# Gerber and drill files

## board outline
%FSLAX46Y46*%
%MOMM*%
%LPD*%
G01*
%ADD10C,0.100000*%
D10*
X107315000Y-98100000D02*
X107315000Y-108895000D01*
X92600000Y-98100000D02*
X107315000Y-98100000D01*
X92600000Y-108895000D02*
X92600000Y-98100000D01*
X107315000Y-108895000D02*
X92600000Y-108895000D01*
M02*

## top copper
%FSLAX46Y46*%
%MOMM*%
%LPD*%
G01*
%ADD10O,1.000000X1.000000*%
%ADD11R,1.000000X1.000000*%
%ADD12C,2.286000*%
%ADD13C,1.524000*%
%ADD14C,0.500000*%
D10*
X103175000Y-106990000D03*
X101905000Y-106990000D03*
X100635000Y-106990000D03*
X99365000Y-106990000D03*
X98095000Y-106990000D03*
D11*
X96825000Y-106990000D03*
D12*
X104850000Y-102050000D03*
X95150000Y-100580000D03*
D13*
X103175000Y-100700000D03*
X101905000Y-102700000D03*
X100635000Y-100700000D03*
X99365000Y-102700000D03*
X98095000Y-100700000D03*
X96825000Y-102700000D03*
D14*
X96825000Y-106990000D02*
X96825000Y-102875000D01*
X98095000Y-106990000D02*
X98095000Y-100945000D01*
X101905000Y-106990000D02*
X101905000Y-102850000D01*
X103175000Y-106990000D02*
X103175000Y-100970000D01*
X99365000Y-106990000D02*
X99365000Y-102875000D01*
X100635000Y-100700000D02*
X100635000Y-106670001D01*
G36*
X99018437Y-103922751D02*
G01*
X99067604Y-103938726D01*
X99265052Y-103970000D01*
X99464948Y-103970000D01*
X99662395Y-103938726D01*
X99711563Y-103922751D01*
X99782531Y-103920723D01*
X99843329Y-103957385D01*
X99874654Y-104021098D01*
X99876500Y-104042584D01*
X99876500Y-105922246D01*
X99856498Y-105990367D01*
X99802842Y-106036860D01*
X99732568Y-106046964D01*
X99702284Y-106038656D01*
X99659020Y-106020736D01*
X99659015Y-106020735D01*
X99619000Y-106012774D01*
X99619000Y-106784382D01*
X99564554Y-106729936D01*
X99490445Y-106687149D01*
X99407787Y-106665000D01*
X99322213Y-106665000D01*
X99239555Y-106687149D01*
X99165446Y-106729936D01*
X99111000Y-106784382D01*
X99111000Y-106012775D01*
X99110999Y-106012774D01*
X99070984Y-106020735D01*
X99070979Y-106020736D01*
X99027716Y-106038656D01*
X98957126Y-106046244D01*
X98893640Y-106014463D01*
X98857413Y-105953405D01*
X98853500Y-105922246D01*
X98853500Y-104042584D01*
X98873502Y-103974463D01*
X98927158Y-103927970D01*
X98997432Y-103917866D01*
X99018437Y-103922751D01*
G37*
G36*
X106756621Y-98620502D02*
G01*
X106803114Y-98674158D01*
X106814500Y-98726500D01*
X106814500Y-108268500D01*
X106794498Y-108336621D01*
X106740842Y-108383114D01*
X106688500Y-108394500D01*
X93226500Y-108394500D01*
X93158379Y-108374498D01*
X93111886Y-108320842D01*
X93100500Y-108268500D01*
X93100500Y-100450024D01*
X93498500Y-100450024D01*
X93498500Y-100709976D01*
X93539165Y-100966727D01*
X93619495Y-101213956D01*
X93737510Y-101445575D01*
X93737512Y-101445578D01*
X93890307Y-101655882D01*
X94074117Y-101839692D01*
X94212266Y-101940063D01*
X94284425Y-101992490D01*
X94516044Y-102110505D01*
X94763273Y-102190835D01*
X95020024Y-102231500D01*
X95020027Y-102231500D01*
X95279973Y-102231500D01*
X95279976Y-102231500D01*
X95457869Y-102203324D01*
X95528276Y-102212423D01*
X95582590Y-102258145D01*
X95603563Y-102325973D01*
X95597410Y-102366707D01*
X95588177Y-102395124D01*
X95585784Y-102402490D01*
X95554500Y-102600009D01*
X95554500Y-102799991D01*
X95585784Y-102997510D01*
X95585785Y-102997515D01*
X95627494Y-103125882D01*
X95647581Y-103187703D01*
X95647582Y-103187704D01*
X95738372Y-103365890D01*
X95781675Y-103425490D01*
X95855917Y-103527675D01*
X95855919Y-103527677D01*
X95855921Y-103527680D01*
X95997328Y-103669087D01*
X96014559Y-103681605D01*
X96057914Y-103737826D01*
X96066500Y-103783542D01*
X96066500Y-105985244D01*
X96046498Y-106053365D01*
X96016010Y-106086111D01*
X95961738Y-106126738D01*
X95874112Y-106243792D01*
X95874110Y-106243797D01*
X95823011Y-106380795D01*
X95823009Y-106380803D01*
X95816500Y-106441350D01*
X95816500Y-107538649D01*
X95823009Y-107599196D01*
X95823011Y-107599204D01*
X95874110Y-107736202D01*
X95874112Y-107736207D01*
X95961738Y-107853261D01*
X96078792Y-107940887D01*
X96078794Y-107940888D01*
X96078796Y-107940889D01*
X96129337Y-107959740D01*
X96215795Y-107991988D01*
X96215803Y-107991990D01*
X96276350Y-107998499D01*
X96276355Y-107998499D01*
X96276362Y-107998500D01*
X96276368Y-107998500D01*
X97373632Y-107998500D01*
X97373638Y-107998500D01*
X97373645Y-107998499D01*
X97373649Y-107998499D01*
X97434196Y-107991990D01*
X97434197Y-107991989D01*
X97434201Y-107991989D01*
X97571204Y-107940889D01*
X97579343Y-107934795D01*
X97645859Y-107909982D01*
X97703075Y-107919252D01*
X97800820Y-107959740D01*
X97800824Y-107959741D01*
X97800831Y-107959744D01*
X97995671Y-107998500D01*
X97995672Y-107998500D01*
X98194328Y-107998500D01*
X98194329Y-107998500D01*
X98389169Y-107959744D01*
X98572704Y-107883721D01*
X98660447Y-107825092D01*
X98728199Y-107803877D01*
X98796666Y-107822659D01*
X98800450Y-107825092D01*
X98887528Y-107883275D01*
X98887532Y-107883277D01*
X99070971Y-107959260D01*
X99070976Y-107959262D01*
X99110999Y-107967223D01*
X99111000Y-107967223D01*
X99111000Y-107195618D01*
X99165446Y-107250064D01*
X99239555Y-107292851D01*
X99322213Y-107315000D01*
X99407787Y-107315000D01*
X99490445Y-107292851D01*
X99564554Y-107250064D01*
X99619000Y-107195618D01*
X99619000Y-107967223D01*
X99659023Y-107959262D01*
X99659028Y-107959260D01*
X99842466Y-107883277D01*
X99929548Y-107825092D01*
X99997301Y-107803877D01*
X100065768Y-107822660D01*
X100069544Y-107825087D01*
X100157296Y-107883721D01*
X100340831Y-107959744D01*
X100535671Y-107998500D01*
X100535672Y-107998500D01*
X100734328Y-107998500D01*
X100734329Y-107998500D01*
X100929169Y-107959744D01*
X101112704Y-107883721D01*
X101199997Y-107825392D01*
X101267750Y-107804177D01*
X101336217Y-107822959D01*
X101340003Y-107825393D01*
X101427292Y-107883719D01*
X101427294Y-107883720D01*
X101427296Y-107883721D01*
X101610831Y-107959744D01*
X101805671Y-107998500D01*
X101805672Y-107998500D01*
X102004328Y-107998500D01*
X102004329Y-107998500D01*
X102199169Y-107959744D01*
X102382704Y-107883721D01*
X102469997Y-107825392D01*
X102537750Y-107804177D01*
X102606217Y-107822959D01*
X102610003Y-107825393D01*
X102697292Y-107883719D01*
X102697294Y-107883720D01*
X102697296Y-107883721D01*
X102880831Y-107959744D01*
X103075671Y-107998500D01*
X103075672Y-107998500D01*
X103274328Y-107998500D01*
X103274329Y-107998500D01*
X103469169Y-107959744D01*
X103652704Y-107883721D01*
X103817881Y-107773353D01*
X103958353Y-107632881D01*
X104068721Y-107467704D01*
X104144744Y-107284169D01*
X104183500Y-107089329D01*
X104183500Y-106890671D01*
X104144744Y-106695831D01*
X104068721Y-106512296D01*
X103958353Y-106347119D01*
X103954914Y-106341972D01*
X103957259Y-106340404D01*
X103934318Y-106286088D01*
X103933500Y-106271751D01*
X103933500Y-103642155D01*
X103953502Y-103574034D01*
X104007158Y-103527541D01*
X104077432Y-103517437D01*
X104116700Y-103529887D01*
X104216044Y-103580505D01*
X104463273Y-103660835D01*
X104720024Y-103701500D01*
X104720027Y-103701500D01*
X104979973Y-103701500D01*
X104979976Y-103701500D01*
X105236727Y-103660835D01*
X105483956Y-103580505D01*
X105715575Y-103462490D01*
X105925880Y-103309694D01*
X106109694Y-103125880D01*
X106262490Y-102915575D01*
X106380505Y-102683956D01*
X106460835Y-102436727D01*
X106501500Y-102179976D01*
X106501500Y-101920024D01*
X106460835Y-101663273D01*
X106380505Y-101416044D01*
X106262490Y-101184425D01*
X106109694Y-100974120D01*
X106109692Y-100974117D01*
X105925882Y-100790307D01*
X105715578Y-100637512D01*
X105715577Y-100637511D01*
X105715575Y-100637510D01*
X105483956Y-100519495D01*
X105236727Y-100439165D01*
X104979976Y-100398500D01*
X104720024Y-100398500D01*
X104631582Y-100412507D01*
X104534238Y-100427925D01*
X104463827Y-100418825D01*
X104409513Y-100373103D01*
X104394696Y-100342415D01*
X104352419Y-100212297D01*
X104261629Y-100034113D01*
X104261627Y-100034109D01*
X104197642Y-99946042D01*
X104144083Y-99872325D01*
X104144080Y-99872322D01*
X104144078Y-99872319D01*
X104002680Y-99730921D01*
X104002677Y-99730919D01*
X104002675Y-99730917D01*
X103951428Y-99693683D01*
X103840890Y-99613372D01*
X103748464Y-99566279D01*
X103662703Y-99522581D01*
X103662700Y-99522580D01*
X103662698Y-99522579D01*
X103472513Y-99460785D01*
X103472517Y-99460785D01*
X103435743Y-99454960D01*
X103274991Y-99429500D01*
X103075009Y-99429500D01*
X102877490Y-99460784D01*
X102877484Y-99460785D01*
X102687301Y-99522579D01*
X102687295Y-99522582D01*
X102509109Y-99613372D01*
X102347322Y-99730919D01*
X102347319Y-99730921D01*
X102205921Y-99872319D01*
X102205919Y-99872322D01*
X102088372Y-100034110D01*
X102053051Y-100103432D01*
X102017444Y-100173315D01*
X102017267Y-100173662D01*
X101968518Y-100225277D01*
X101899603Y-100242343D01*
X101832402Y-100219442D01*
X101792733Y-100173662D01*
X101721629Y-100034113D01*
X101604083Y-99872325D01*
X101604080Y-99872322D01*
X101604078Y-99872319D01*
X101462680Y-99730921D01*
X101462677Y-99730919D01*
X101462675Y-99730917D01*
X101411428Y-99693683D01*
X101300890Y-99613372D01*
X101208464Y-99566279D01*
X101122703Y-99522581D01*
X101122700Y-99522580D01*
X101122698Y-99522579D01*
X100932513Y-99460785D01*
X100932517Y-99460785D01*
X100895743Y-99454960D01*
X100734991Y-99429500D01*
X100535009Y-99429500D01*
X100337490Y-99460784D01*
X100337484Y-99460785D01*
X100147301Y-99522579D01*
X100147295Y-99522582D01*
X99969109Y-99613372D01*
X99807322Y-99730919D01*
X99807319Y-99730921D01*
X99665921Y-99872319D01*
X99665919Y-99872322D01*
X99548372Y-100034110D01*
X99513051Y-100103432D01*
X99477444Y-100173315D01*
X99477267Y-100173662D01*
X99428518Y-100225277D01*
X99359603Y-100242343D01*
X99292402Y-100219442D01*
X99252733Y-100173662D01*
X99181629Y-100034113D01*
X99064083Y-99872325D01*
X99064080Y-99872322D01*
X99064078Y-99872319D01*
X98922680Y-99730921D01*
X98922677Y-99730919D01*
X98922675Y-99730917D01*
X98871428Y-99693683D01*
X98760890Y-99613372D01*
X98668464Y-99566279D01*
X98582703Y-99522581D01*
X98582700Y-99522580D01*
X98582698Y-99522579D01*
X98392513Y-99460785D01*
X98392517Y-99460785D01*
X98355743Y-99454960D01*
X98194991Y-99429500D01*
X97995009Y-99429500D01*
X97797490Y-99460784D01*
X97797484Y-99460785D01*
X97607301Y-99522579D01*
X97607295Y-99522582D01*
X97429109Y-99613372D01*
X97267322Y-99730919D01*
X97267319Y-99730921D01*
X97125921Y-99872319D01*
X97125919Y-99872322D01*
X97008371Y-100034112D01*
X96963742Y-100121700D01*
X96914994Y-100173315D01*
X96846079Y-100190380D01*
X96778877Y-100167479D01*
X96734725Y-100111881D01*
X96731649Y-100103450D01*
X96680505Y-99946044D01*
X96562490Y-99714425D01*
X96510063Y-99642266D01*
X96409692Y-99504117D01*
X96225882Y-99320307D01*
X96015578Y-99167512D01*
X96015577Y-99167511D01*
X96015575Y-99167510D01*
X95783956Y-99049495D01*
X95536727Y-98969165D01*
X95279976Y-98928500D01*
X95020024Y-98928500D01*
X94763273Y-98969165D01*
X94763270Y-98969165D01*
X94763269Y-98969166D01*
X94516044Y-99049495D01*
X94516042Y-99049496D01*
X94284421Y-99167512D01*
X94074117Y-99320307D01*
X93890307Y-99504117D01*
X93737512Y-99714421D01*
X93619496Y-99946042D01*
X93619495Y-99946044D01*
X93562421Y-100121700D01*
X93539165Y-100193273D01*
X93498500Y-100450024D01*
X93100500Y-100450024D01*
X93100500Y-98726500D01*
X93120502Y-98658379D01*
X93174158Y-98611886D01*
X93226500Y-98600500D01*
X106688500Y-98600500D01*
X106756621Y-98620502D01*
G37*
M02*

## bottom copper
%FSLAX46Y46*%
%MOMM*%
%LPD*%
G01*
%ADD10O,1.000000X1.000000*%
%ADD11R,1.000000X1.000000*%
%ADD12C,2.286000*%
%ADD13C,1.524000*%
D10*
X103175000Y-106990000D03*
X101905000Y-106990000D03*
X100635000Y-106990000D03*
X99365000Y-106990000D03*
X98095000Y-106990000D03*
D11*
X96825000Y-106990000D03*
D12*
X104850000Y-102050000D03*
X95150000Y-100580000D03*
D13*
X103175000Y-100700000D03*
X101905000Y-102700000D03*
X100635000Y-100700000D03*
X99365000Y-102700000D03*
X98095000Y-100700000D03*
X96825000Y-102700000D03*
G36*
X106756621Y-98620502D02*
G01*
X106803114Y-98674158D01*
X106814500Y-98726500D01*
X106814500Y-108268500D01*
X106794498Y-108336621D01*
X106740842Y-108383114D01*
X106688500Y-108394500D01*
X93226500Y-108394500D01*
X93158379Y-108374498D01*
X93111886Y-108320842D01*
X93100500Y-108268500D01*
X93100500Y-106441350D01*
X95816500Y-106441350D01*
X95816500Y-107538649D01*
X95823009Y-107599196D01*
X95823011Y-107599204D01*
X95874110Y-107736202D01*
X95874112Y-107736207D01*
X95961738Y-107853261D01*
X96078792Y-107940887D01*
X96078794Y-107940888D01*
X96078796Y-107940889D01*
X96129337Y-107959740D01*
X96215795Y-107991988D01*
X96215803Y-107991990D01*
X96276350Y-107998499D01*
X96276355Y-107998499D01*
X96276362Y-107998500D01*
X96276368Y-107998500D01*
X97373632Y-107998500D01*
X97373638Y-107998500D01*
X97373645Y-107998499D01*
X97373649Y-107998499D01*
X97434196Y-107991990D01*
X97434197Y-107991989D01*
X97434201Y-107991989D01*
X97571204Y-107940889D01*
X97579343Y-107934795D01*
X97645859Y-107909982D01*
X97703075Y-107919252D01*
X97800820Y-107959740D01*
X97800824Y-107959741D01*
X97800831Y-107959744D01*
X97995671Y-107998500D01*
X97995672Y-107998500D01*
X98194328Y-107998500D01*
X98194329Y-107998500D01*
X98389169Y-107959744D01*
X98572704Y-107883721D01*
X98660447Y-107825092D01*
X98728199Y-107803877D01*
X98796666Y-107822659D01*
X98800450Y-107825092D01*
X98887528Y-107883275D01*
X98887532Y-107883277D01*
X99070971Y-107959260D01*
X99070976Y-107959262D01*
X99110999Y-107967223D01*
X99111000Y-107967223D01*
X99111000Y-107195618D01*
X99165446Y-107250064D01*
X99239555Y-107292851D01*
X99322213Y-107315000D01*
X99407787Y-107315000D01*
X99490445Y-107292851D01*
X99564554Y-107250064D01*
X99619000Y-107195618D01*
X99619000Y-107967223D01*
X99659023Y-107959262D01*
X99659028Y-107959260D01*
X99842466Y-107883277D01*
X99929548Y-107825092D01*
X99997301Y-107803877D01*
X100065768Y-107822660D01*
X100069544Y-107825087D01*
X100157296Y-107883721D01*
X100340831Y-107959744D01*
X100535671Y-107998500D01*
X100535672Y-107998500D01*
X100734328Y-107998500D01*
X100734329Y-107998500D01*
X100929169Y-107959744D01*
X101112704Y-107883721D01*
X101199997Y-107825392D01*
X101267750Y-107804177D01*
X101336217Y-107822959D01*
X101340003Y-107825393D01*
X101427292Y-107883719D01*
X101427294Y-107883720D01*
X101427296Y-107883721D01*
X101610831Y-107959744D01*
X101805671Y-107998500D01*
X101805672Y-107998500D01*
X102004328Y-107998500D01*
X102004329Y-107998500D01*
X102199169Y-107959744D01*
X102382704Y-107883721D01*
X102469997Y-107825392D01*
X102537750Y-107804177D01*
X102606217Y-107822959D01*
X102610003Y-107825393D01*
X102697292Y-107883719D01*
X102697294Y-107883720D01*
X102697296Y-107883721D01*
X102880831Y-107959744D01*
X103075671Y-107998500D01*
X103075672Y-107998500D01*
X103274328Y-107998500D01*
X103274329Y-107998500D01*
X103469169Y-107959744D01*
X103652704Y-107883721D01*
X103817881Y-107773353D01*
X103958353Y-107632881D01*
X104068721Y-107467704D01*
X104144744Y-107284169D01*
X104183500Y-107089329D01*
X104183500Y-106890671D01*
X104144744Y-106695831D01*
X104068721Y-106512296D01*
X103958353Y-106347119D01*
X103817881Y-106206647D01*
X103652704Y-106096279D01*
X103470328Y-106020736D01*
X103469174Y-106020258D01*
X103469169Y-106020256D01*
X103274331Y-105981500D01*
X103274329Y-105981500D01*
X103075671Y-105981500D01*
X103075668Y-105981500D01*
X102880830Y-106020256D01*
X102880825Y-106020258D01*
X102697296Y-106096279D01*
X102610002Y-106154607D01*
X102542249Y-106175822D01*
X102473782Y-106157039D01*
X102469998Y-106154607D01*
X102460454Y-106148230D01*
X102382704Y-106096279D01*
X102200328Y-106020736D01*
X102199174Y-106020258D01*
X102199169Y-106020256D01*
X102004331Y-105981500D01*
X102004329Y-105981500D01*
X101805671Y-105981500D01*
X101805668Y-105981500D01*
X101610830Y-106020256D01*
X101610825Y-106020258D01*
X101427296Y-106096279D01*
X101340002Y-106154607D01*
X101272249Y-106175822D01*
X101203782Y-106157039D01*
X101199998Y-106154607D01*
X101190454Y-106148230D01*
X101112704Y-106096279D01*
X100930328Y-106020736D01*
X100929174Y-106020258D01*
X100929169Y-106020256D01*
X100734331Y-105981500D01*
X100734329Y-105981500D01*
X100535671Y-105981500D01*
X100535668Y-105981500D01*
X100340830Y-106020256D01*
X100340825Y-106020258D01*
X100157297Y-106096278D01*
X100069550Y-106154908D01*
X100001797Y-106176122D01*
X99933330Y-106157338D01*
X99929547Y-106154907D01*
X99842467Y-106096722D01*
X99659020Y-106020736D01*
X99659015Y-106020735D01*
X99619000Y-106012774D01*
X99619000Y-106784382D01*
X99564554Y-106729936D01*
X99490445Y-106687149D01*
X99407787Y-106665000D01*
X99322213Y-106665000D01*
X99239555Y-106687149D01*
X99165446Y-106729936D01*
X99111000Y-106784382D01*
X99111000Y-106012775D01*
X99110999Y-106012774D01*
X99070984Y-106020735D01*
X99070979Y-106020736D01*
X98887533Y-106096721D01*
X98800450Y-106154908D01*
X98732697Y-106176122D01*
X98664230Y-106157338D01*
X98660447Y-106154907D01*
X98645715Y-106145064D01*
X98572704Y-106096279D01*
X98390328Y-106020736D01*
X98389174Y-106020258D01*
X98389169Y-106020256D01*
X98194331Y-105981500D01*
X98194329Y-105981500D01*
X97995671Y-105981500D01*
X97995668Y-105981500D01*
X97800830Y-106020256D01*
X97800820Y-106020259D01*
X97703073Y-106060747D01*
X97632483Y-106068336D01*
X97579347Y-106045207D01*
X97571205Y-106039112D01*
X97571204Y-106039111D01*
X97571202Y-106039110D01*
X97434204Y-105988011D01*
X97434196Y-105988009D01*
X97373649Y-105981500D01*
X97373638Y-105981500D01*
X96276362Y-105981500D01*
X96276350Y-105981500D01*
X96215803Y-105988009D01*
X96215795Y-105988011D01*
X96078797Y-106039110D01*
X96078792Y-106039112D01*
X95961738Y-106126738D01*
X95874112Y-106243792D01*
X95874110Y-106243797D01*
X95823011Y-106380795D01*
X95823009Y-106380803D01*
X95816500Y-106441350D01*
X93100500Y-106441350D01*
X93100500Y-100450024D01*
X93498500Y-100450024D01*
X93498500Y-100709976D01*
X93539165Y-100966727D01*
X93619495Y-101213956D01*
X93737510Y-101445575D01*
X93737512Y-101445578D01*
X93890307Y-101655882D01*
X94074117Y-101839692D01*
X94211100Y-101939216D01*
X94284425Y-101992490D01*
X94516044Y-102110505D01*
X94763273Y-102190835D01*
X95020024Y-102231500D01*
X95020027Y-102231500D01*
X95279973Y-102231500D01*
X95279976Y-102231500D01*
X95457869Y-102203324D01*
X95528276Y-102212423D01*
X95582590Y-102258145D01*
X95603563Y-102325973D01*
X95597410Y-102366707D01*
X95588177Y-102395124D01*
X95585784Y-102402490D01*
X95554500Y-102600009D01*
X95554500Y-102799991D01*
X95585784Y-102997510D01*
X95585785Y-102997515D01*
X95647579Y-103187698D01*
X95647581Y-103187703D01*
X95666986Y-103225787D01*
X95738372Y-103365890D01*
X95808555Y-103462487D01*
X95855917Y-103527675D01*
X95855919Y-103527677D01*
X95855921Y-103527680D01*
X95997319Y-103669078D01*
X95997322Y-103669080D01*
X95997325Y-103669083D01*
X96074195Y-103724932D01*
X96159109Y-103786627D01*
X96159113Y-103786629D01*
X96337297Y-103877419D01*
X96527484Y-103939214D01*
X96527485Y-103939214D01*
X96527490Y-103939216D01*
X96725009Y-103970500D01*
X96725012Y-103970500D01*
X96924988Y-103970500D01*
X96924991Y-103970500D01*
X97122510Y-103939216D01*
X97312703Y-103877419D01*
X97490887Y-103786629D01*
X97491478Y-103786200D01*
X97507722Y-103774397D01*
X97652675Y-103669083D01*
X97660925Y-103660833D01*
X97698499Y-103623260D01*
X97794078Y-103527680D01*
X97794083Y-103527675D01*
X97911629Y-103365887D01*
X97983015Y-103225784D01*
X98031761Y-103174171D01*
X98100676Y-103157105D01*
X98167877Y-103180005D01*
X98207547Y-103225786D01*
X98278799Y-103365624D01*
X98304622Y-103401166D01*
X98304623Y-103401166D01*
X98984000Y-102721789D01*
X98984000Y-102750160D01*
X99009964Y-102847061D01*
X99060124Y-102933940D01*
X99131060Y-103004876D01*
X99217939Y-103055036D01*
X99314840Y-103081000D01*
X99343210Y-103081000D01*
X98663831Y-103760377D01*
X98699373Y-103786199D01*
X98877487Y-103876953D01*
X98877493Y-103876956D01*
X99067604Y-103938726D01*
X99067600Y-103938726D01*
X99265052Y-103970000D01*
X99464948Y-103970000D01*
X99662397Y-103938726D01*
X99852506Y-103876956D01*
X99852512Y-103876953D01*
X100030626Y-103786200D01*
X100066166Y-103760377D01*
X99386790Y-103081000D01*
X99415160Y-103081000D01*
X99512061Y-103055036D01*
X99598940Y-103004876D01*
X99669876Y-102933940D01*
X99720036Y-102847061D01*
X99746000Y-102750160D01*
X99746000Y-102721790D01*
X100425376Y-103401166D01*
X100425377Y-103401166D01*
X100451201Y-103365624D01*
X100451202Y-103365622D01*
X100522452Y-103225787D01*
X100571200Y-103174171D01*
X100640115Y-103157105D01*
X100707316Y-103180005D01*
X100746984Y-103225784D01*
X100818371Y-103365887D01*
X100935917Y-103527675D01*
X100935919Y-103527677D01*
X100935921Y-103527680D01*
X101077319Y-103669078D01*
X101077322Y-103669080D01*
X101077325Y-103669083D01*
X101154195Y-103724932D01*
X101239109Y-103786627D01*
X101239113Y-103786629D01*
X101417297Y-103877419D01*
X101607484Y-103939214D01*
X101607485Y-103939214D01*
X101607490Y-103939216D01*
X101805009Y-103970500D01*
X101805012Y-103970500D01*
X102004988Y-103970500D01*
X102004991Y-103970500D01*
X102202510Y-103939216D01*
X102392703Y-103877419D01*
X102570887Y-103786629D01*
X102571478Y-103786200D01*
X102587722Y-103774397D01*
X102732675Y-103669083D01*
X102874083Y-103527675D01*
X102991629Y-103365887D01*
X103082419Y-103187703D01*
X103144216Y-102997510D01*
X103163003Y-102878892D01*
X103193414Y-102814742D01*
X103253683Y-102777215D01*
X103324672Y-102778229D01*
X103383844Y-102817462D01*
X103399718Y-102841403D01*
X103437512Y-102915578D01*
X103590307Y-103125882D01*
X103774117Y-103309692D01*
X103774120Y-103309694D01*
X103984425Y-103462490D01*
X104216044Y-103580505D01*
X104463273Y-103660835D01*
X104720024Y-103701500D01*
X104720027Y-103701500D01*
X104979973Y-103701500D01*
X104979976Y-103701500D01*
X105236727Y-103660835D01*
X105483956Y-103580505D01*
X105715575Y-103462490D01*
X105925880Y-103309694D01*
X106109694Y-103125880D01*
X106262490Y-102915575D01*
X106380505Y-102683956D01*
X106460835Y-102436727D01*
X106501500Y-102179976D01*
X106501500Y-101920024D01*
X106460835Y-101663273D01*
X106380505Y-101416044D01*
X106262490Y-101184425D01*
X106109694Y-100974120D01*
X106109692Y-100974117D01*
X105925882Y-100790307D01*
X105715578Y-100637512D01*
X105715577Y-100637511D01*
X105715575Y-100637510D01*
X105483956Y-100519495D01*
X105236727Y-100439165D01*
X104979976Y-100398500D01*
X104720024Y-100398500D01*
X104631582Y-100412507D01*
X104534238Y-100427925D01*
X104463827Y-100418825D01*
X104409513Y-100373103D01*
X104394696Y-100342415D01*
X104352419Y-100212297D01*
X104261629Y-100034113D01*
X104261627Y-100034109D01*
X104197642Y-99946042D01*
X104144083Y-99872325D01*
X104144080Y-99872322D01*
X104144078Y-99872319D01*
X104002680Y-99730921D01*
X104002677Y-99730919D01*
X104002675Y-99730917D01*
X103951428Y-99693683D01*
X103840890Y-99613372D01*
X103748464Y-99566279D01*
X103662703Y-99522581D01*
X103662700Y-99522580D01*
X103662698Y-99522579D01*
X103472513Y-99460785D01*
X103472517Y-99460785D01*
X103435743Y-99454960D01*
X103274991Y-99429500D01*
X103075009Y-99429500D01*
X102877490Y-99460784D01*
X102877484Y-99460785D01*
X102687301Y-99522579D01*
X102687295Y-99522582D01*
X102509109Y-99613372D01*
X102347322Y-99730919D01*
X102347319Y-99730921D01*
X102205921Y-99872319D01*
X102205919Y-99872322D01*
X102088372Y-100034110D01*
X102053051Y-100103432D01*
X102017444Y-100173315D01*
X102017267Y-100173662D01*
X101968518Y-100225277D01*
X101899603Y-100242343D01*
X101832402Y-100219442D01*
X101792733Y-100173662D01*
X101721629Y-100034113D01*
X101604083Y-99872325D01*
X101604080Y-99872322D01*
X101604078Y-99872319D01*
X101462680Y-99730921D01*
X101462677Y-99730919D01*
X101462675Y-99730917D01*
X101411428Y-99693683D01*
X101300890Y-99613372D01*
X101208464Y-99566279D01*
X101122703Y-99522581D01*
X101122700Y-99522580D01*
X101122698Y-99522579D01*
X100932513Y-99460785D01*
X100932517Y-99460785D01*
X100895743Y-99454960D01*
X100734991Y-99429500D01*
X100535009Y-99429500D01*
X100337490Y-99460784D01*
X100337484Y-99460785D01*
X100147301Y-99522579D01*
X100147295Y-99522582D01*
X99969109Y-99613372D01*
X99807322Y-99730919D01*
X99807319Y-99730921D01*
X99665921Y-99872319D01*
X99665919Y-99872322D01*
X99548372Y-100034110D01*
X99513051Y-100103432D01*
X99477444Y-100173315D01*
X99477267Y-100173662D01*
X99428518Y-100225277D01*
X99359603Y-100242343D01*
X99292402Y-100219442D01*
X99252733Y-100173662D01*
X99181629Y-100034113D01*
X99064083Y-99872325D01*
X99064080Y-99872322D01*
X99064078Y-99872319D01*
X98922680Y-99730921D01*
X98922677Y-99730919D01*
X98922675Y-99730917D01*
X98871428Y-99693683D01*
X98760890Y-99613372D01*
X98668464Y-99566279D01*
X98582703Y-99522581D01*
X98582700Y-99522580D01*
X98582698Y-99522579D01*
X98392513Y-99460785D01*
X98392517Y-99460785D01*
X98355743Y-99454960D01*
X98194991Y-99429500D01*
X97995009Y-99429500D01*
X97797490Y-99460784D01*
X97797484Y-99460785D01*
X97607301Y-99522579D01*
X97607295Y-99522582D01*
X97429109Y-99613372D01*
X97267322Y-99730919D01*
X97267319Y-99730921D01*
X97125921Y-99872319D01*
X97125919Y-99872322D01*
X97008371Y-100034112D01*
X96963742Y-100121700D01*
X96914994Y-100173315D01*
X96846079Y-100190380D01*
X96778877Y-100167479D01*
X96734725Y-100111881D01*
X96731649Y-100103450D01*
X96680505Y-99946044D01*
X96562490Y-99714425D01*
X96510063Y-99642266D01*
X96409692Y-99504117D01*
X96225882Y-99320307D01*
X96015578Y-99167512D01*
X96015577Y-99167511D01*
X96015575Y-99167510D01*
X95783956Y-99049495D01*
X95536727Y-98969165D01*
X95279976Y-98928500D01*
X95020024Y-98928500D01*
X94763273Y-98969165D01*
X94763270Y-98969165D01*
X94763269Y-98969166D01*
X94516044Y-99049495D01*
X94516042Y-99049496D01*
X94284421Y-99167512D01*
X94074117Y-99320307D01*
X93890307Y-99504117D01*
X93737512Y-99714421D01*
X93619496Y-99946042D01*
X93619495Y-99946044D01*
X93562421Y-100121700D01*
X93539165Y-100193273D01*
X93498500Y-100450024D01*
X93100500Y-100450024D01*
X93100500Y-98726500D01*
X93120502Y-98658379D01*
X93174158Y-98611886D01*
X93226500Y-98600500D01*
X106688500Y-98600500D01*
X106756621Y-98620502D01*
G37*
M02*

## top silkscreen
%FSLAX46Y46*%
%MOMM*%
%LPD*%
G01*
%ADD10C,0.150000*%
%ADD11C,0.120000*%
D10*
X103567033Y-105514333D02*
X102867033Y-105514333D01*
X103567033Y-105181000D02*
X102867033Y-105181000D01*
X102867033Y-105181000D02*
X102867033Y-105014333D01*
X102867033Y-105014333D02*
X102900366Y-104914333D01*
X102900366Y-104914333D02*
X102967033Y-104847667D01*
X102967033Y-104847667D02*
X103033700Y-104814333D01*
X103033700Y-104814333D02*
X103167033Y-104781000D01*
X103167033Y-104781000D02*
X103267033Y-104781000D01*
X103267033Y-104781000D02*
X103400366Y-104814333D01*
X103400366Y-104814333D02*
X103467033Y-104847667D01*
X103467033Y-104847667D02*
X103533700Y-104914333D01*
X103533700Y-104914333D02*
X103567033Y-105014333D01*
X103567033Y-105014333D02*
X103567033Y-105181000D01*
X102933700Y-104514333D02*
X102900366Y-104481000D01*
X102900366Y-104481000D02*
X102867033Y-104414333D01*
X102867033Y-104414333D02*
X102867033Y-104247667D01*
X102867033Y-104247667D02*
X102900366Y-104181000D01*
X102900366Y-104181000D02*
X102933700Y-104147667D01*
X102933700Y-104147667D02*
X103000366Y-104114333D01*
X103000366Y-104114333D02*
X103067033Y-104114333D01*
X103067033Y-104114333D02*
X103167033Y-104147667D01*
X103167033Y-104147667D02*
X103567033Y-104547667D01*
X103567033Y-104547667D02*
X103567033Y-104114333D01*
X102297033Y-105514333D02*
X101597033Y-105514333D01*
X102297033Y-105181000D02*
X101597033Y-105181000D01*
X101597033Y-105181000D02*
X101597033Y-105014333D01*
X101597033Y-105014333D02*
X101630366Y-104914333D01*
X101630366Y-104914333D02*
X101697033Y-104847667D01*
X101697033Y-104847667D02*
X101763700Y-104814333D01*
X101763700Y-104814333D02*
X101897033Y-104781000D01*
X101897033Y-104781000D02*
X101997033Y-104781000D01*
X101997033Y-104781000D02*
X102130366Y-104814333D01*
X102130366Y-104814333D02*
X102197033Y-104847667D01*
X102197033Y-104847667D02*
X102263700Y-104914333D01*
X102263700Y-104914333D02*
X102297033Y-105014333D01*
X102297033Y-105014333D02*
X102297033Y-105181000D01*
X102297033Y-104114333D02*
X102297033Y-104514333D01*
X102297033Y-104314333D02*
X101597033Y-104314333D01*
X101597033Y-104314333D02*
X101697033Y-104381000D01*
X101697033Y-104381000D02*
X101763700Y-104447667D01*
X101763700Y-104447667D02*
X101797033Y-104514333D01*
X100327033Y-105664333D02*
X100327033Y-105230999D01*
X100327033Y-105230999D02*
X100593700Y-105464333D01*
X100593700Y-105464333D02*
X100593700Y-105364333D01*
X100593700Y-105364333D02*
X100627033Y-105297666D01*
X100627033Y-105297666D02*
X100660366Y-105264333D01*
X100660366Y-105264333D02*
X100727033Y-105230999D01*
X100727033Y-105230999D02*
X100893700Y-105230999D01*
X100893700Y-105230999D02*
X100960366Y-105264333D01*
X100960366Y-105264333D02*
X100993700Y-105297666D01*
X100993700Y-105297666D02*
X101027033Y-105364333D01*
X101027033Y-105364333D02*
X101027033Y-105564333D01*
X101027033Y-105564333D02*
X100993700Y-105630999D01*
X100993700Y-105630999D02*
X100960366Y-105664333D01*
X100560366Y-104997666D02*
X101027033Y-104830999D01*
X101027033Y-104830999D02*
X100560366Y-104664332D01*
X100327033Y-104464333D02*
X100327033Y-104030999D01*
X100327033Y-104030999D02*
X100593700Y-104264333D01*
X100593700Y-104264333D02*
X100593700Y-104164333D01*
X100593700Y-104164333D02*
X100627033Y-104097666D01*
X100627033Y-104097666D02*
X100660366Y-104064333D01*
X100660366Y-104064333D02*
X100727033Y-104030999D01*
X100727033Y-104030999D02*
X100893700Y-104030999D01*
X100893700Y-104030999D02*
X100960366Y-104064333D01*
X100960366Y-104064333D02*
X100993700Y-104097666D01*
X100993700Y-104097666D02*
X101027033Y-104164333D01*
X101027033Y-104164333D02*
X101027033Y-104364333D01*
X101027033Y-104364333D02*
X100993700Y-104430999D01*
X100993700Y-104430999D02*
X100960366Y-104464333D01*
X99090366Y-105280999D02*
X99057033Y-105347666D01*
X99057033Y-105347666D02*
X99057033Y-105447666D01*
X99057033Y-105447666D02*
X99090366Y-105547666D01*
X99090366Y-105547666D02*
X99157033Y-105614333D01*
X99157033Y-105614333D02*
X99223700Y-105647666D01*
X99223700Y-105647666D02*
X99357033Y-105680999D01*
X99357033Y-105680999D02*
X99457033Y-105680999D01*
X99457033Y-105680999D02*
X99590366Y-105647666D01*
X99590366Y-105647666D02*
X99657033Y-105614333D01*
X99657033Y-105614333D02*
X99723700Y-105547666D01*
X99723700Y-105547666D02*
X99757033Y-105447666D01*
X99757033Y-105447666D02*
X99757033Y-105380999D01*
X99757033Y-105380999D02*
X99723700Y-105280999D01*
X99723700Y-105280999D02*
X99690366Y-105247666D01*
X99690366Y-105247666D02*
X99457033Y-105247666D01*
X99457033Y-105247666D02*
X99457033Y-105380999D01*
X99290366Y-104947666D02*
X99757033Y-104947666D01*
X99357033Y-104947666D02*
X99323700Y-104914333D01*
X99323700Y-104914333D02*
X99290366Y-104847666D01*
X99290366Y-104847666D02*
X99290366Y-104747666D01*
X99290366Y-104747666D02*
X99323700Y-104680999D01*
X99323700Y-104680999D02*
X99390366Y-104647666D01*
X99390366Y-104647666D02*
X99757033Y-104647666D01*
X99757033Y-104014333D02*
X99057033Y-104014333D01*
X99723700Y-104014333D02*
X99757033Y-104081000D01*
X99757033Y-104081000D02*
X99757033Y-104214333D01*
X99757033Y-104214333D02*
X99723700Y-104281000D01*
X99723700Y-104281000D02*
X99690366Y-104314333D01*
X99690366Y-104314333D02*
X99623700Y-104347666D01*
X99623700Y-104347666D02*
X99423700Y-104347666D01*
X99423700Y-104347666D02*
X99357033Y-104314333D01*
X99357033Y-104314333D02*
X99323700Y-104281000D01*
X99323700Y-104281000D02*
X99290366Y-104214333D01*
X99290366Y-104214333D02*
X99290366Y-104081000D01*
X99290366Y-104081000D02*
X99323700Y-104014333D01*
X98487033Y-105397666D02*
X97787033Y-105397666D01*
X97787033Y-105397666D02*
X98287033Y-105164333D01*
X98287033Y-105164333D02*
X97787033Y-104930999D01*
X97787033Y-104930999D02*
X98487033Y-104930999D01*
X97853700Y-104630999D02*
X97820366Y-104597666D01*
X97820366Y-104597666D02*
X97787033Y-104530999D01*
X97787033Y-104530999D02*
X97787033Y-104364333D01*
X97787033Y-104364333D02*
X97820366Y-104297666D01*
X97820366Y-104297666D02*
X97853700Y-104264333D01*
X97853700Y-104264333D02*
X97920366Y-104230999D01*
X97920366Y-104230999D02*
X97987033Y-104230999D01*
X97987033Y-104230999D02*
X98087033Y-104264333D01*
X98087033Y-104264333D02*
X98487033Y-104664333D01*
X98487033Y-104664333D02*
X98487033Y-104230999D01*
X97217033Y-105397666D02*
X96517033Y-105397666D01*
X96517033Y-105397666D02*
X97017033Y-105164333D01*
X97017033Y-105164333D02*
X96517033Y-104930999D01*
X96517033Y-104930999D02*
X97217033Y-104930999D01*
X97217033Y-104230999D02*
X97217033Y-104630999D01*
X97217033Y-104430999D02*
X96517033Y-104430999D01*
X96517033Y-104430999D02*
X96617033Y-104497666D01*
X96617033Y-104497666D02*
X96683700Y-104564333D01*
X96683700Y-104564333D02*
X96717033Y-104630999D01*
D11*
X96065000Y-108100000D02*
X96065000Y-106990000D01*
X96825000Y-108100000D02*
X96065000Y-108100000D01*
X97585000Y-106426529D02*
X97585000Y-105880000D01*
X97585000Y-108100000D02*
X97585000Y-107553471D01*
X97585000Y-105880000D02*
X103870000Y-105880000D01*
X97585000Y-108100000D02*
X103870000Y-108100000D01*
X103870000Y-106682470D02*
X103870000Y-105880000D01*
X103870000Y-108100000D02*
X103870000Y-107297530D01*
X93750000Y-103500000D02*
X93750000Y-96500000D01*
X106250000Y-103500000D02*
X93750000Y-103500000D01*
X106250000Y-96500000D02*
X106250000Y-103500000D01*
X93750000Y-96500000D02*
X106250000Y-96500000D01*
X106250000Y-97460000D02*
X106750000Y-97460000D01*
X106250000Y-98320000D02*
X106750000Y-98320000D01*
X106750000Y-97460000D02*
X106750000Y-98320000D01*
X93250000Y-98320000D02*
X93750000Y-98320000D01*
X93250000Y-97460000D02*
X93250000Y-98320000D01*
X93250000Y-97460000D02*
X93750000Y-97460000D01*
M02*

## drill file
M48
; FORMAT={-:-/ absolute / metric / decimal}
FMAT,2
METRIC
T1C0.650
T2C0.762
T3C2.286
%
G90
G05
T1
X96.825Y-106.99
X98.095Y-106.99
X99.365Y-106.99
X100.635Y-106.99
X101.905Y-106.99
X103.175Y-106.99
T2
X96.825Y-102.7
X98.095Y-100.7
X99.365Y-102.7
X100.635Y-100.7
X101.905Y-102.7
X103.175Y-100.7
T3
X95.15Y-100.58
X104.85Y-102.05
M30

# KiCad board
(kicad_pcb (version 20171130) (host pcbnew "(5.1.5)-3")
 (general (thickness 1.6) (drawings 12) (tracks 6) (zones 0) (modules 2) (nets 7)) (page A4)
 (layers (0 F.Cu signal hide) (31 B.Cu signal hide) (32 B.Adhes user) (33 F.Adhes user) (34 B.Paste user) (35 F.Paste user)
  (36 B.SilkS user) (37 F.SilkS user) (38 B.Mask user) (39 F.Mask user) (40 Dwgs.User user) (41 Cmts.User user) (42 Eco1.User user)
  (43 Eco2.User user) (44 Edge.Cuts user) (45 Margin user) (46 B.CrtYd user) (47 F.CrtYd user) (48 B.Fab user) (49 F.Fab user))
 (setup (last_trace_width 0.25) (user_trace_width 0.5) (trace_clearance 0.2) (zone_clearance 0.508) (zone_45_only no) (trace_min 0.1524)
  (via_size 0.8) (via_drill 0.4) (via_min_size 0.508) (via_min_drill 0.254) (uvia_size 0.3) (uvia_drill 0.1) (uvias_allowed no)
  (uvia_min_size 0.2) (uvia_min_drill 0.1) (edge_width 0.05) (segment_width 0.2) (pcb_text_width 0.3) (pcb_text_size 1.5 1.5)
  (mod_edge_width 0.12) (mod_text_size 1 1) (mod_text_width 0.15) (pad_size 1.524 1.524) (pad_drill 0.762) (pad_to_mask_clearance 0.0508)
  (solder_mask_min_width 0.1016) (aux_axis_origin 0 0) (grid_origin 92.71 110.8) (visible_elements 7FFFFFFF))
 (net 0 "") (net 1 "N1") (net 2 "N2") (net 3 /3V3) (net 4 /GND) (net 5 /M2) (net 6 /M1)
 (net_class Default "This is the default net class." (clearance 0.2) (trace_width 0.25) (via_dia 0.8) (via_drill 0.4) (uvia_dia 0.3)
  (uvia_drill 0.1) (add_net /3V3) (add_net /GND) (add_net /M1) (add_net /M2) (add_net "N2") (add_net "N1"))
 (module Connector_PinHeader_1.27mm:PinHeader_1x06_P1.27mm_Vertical (layer F.Cu) (at 96.825 106.99 90)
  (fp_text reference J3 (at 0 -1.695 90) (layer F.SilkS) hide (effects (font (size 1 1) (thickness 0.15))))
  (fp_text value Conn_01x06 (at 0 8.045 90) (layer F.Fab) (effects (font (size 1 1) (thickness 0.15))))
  (fp_line (start -1.11 -0.76) (end 0 -0.76) (layer F.SilkS) (width 0.12))
  (fp_line (start -1.11 0) (end -1.11 -0.76) (layer F.SilkS) (width 0.12))
  (fp_line (start 0.563471 0.76) (end 1.11 0.76) (layer F.SilkS) (width 0.12))
  (fp_line (start -1.11 0.76) (end -0.563471 0.76) (layer F.SilkS) (width 0.12))
  (fp_line (start 1.11 0.76) (end 1.11 7.045) (layer F.SilkS) (width 0.12))
  (fp_line (start -1.11 0.76) (end -1.11 7.045) (layer F.SilkS) (width 0.12))
  (fp_line (start 0.30753 7.045) (end 1.11 7.045) (layer F.SilkS) (width 0.12))
  (fp_line (start -1.11 7.045) (end -0.30753 7.045) (layer F.SilkS) (width 0.12))
  (pad 6 thru_hole oval (at 0 6.35 90) (size 1 1) (drill 0.65) (layers *.Cu *.Mask) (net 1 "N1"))
  (pad 5 thru_hole oval (at 0 5.08 90) (size 1 1) (drill 0.65) (layers *.Cu *.Mask) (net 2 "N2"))
  (pad 4 thru_hole oval (at 0 3.81 90) (size 1 1) (drill 0.65) (layers *.Cu *.Mask) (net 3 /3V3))
  (pad 3 thru_hole oval (at 0 2.54 90) (size 1 1) (drill 0.65) (layers *.Cu *.Mask) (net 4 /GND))
  (pad 2 thru_hole oval (at 0 1.27 90) (size 1 1) (drill 0.65) (layers *.Cu *.Mask) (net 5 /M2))
  (pad 1 thru_hole rect (at 0 0 90) (size 1 1) (drill 0.65) (layers *.Cu *.Mask) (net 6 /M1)))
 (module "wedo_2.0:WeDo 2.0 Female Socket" (layer F.Cu) (at 100 100)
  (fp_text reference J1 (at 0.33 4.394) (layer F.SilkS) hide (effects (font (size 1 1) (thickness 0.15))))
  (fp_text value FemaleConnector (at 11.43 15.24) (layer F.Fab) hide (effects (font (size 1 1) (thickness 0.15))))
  (fp_line (start -6.25 3.5) (end -6.25 -3.5) (layer F.SilkS) (width 0.12))
  (fp_line (start 6.25 3.5) (end -6.25 3.5) (layer F.SilkS) (width 0.12))
  (fp_line (start 6.25 -3.5) (end 6.25 3.5) (layer F.SilkS) (width 0.12))
  (fp_line (start -6.25 -3.5) (end 6.25 -3.5) (layer F.SilkS) (width 0.12))
  (fp_line (start 6.25 -2.54) (end 6.75 -2.54) (layer F.SilkS) (width 0.12))
  (fp_line (start 6.25 -1.68) (end 6.75 -1.68) (layer F.SilkS) (width 0.12))
  (fp_line (start 6.75 -2.54) (end 6.75 -1.68) (layer F.SilkS) (width 0.12))
  (fp_line (start -6.75 -1.68) (end -6.25 -1.68) (layer F.SilkS) (width 0.12))
  (fp_line (start -6.75 -2.54) (end -6.75 -1.68) (layer F.SilkS) (width 0.12))
  (fp_line (start -6.75 -2.54) (end -6.25 -2.54) (layer F.SilkS) (width 0.12))
  (pad "" thru_hole circle (at 4.85 2.05) (size 2.286 2.286) (drill 2.286) (layers *.Cu *.Mask))
  (pad "" thru_hole circle (at -4.85 0.58) (size 2.286 2.286) (drill 2.286) (layers *.Cu *.Mask))
  (pad 6 thru_hole circle (at 3.175 0.7) (size 1.524 1.524) (drill 0.762) (layers *.Cu *.Mask) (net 1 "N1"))
  (pad 5 thru_hole circle (at 1.905 2.7) (size 1.524 1.524) (drill 0.762) (layers *.Cu *.Mask) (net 2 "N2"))
  (pad 4 thru_hole circle (at 0.635 0.7) (size 1.524 1.524) (drill 0.762) (layers *.Cu *.Mask) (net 3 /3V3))
  (pad 3 thru_hole circle (at -0.635 2.7) (size 1.524 1.524) (drill 0.762) (layers *.Cu *.Mask) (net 4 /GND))
  (pad 2 thru_hole circle (at -1.905 0.7) (size 1.524 1.524) (drill 0.762) (layers *.Cu *.Mask) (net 5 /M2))
  (pad 1 thru_hole circle (at -3.175 2.7) (size 1.524 1.524) (drill 0.762) (layers *.Cu *.Mask) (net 6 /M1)))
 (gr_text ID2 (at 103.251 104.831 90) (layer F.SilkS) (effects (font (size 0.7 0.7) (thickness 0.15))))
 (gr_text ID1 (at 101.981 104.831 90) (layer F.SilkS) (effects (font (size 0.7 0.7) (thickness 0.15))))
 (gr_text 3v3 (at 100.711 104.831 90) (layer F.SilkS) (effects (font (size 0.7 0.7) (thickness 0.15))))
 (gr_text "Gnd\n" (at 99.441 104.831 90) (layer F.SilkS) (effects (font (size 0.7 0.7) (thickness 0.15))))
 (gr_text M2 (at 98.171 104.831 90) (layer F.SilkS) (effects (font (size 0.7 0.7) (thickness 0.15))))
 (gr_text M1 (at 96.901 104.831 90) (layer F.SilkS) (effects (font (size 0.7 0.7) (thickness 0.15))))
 (gr_line (start 107.315 98.1) (end 107.315 108.895) (layer Edge.Cuts) (width 0.1))
 (gr_line (start 92.6 98.1) (end 107.315 98.1) (layer Edge.Cuts) (width 0.1))
 (gr_line (start 92.6 108.895) (end 92.6 98.1) (layer Edge.Cuts) (width 0.1))
 (gr_line (start 107.315 108.895) (end 92.6 108.895) (layer Edge.Cuts) (width 0.1))
 (segment (start 96.825 106.99) (end 96.825 102.875) (width 0.5) (layer F.Cu) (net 6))
 (segment (start 98.095 106.99) (end 98.095 100.945) (width 0.5) (layer F.Cu) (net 5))
 (segment (start 101.905 106.99) (end 101.905 102.85) (width 0.5) (layer F.Cu) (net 2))
 (segment (start 103.175 106.99) (end 103.175 100.97) (width 0.5) (layer F.Cu) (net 1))
 (segment (start 99.365 106.99) (end 99.365 102.875) (width 0.5) (layer F.Cu) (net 4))
 (segment (start 100.635 100.7) (end 100.635 106.670001) (width 0.5) (layer F.Cu) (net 3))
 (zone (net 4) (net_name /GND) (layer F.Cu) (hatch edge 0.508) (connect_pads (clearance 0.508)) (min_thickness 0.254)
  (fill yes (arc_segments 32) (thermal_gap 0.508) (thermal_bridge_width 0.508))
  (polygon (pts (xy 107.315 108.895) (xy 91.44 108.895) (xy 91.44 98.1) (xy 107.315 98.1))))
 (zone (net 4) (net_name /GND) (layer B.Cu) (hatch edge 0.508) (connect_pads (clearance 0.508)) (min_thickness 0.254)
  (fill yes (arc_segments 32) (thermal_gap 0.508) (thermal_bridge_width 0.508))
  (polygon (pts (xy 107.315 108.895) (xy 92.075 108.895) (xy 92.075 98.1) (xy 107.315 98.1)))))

